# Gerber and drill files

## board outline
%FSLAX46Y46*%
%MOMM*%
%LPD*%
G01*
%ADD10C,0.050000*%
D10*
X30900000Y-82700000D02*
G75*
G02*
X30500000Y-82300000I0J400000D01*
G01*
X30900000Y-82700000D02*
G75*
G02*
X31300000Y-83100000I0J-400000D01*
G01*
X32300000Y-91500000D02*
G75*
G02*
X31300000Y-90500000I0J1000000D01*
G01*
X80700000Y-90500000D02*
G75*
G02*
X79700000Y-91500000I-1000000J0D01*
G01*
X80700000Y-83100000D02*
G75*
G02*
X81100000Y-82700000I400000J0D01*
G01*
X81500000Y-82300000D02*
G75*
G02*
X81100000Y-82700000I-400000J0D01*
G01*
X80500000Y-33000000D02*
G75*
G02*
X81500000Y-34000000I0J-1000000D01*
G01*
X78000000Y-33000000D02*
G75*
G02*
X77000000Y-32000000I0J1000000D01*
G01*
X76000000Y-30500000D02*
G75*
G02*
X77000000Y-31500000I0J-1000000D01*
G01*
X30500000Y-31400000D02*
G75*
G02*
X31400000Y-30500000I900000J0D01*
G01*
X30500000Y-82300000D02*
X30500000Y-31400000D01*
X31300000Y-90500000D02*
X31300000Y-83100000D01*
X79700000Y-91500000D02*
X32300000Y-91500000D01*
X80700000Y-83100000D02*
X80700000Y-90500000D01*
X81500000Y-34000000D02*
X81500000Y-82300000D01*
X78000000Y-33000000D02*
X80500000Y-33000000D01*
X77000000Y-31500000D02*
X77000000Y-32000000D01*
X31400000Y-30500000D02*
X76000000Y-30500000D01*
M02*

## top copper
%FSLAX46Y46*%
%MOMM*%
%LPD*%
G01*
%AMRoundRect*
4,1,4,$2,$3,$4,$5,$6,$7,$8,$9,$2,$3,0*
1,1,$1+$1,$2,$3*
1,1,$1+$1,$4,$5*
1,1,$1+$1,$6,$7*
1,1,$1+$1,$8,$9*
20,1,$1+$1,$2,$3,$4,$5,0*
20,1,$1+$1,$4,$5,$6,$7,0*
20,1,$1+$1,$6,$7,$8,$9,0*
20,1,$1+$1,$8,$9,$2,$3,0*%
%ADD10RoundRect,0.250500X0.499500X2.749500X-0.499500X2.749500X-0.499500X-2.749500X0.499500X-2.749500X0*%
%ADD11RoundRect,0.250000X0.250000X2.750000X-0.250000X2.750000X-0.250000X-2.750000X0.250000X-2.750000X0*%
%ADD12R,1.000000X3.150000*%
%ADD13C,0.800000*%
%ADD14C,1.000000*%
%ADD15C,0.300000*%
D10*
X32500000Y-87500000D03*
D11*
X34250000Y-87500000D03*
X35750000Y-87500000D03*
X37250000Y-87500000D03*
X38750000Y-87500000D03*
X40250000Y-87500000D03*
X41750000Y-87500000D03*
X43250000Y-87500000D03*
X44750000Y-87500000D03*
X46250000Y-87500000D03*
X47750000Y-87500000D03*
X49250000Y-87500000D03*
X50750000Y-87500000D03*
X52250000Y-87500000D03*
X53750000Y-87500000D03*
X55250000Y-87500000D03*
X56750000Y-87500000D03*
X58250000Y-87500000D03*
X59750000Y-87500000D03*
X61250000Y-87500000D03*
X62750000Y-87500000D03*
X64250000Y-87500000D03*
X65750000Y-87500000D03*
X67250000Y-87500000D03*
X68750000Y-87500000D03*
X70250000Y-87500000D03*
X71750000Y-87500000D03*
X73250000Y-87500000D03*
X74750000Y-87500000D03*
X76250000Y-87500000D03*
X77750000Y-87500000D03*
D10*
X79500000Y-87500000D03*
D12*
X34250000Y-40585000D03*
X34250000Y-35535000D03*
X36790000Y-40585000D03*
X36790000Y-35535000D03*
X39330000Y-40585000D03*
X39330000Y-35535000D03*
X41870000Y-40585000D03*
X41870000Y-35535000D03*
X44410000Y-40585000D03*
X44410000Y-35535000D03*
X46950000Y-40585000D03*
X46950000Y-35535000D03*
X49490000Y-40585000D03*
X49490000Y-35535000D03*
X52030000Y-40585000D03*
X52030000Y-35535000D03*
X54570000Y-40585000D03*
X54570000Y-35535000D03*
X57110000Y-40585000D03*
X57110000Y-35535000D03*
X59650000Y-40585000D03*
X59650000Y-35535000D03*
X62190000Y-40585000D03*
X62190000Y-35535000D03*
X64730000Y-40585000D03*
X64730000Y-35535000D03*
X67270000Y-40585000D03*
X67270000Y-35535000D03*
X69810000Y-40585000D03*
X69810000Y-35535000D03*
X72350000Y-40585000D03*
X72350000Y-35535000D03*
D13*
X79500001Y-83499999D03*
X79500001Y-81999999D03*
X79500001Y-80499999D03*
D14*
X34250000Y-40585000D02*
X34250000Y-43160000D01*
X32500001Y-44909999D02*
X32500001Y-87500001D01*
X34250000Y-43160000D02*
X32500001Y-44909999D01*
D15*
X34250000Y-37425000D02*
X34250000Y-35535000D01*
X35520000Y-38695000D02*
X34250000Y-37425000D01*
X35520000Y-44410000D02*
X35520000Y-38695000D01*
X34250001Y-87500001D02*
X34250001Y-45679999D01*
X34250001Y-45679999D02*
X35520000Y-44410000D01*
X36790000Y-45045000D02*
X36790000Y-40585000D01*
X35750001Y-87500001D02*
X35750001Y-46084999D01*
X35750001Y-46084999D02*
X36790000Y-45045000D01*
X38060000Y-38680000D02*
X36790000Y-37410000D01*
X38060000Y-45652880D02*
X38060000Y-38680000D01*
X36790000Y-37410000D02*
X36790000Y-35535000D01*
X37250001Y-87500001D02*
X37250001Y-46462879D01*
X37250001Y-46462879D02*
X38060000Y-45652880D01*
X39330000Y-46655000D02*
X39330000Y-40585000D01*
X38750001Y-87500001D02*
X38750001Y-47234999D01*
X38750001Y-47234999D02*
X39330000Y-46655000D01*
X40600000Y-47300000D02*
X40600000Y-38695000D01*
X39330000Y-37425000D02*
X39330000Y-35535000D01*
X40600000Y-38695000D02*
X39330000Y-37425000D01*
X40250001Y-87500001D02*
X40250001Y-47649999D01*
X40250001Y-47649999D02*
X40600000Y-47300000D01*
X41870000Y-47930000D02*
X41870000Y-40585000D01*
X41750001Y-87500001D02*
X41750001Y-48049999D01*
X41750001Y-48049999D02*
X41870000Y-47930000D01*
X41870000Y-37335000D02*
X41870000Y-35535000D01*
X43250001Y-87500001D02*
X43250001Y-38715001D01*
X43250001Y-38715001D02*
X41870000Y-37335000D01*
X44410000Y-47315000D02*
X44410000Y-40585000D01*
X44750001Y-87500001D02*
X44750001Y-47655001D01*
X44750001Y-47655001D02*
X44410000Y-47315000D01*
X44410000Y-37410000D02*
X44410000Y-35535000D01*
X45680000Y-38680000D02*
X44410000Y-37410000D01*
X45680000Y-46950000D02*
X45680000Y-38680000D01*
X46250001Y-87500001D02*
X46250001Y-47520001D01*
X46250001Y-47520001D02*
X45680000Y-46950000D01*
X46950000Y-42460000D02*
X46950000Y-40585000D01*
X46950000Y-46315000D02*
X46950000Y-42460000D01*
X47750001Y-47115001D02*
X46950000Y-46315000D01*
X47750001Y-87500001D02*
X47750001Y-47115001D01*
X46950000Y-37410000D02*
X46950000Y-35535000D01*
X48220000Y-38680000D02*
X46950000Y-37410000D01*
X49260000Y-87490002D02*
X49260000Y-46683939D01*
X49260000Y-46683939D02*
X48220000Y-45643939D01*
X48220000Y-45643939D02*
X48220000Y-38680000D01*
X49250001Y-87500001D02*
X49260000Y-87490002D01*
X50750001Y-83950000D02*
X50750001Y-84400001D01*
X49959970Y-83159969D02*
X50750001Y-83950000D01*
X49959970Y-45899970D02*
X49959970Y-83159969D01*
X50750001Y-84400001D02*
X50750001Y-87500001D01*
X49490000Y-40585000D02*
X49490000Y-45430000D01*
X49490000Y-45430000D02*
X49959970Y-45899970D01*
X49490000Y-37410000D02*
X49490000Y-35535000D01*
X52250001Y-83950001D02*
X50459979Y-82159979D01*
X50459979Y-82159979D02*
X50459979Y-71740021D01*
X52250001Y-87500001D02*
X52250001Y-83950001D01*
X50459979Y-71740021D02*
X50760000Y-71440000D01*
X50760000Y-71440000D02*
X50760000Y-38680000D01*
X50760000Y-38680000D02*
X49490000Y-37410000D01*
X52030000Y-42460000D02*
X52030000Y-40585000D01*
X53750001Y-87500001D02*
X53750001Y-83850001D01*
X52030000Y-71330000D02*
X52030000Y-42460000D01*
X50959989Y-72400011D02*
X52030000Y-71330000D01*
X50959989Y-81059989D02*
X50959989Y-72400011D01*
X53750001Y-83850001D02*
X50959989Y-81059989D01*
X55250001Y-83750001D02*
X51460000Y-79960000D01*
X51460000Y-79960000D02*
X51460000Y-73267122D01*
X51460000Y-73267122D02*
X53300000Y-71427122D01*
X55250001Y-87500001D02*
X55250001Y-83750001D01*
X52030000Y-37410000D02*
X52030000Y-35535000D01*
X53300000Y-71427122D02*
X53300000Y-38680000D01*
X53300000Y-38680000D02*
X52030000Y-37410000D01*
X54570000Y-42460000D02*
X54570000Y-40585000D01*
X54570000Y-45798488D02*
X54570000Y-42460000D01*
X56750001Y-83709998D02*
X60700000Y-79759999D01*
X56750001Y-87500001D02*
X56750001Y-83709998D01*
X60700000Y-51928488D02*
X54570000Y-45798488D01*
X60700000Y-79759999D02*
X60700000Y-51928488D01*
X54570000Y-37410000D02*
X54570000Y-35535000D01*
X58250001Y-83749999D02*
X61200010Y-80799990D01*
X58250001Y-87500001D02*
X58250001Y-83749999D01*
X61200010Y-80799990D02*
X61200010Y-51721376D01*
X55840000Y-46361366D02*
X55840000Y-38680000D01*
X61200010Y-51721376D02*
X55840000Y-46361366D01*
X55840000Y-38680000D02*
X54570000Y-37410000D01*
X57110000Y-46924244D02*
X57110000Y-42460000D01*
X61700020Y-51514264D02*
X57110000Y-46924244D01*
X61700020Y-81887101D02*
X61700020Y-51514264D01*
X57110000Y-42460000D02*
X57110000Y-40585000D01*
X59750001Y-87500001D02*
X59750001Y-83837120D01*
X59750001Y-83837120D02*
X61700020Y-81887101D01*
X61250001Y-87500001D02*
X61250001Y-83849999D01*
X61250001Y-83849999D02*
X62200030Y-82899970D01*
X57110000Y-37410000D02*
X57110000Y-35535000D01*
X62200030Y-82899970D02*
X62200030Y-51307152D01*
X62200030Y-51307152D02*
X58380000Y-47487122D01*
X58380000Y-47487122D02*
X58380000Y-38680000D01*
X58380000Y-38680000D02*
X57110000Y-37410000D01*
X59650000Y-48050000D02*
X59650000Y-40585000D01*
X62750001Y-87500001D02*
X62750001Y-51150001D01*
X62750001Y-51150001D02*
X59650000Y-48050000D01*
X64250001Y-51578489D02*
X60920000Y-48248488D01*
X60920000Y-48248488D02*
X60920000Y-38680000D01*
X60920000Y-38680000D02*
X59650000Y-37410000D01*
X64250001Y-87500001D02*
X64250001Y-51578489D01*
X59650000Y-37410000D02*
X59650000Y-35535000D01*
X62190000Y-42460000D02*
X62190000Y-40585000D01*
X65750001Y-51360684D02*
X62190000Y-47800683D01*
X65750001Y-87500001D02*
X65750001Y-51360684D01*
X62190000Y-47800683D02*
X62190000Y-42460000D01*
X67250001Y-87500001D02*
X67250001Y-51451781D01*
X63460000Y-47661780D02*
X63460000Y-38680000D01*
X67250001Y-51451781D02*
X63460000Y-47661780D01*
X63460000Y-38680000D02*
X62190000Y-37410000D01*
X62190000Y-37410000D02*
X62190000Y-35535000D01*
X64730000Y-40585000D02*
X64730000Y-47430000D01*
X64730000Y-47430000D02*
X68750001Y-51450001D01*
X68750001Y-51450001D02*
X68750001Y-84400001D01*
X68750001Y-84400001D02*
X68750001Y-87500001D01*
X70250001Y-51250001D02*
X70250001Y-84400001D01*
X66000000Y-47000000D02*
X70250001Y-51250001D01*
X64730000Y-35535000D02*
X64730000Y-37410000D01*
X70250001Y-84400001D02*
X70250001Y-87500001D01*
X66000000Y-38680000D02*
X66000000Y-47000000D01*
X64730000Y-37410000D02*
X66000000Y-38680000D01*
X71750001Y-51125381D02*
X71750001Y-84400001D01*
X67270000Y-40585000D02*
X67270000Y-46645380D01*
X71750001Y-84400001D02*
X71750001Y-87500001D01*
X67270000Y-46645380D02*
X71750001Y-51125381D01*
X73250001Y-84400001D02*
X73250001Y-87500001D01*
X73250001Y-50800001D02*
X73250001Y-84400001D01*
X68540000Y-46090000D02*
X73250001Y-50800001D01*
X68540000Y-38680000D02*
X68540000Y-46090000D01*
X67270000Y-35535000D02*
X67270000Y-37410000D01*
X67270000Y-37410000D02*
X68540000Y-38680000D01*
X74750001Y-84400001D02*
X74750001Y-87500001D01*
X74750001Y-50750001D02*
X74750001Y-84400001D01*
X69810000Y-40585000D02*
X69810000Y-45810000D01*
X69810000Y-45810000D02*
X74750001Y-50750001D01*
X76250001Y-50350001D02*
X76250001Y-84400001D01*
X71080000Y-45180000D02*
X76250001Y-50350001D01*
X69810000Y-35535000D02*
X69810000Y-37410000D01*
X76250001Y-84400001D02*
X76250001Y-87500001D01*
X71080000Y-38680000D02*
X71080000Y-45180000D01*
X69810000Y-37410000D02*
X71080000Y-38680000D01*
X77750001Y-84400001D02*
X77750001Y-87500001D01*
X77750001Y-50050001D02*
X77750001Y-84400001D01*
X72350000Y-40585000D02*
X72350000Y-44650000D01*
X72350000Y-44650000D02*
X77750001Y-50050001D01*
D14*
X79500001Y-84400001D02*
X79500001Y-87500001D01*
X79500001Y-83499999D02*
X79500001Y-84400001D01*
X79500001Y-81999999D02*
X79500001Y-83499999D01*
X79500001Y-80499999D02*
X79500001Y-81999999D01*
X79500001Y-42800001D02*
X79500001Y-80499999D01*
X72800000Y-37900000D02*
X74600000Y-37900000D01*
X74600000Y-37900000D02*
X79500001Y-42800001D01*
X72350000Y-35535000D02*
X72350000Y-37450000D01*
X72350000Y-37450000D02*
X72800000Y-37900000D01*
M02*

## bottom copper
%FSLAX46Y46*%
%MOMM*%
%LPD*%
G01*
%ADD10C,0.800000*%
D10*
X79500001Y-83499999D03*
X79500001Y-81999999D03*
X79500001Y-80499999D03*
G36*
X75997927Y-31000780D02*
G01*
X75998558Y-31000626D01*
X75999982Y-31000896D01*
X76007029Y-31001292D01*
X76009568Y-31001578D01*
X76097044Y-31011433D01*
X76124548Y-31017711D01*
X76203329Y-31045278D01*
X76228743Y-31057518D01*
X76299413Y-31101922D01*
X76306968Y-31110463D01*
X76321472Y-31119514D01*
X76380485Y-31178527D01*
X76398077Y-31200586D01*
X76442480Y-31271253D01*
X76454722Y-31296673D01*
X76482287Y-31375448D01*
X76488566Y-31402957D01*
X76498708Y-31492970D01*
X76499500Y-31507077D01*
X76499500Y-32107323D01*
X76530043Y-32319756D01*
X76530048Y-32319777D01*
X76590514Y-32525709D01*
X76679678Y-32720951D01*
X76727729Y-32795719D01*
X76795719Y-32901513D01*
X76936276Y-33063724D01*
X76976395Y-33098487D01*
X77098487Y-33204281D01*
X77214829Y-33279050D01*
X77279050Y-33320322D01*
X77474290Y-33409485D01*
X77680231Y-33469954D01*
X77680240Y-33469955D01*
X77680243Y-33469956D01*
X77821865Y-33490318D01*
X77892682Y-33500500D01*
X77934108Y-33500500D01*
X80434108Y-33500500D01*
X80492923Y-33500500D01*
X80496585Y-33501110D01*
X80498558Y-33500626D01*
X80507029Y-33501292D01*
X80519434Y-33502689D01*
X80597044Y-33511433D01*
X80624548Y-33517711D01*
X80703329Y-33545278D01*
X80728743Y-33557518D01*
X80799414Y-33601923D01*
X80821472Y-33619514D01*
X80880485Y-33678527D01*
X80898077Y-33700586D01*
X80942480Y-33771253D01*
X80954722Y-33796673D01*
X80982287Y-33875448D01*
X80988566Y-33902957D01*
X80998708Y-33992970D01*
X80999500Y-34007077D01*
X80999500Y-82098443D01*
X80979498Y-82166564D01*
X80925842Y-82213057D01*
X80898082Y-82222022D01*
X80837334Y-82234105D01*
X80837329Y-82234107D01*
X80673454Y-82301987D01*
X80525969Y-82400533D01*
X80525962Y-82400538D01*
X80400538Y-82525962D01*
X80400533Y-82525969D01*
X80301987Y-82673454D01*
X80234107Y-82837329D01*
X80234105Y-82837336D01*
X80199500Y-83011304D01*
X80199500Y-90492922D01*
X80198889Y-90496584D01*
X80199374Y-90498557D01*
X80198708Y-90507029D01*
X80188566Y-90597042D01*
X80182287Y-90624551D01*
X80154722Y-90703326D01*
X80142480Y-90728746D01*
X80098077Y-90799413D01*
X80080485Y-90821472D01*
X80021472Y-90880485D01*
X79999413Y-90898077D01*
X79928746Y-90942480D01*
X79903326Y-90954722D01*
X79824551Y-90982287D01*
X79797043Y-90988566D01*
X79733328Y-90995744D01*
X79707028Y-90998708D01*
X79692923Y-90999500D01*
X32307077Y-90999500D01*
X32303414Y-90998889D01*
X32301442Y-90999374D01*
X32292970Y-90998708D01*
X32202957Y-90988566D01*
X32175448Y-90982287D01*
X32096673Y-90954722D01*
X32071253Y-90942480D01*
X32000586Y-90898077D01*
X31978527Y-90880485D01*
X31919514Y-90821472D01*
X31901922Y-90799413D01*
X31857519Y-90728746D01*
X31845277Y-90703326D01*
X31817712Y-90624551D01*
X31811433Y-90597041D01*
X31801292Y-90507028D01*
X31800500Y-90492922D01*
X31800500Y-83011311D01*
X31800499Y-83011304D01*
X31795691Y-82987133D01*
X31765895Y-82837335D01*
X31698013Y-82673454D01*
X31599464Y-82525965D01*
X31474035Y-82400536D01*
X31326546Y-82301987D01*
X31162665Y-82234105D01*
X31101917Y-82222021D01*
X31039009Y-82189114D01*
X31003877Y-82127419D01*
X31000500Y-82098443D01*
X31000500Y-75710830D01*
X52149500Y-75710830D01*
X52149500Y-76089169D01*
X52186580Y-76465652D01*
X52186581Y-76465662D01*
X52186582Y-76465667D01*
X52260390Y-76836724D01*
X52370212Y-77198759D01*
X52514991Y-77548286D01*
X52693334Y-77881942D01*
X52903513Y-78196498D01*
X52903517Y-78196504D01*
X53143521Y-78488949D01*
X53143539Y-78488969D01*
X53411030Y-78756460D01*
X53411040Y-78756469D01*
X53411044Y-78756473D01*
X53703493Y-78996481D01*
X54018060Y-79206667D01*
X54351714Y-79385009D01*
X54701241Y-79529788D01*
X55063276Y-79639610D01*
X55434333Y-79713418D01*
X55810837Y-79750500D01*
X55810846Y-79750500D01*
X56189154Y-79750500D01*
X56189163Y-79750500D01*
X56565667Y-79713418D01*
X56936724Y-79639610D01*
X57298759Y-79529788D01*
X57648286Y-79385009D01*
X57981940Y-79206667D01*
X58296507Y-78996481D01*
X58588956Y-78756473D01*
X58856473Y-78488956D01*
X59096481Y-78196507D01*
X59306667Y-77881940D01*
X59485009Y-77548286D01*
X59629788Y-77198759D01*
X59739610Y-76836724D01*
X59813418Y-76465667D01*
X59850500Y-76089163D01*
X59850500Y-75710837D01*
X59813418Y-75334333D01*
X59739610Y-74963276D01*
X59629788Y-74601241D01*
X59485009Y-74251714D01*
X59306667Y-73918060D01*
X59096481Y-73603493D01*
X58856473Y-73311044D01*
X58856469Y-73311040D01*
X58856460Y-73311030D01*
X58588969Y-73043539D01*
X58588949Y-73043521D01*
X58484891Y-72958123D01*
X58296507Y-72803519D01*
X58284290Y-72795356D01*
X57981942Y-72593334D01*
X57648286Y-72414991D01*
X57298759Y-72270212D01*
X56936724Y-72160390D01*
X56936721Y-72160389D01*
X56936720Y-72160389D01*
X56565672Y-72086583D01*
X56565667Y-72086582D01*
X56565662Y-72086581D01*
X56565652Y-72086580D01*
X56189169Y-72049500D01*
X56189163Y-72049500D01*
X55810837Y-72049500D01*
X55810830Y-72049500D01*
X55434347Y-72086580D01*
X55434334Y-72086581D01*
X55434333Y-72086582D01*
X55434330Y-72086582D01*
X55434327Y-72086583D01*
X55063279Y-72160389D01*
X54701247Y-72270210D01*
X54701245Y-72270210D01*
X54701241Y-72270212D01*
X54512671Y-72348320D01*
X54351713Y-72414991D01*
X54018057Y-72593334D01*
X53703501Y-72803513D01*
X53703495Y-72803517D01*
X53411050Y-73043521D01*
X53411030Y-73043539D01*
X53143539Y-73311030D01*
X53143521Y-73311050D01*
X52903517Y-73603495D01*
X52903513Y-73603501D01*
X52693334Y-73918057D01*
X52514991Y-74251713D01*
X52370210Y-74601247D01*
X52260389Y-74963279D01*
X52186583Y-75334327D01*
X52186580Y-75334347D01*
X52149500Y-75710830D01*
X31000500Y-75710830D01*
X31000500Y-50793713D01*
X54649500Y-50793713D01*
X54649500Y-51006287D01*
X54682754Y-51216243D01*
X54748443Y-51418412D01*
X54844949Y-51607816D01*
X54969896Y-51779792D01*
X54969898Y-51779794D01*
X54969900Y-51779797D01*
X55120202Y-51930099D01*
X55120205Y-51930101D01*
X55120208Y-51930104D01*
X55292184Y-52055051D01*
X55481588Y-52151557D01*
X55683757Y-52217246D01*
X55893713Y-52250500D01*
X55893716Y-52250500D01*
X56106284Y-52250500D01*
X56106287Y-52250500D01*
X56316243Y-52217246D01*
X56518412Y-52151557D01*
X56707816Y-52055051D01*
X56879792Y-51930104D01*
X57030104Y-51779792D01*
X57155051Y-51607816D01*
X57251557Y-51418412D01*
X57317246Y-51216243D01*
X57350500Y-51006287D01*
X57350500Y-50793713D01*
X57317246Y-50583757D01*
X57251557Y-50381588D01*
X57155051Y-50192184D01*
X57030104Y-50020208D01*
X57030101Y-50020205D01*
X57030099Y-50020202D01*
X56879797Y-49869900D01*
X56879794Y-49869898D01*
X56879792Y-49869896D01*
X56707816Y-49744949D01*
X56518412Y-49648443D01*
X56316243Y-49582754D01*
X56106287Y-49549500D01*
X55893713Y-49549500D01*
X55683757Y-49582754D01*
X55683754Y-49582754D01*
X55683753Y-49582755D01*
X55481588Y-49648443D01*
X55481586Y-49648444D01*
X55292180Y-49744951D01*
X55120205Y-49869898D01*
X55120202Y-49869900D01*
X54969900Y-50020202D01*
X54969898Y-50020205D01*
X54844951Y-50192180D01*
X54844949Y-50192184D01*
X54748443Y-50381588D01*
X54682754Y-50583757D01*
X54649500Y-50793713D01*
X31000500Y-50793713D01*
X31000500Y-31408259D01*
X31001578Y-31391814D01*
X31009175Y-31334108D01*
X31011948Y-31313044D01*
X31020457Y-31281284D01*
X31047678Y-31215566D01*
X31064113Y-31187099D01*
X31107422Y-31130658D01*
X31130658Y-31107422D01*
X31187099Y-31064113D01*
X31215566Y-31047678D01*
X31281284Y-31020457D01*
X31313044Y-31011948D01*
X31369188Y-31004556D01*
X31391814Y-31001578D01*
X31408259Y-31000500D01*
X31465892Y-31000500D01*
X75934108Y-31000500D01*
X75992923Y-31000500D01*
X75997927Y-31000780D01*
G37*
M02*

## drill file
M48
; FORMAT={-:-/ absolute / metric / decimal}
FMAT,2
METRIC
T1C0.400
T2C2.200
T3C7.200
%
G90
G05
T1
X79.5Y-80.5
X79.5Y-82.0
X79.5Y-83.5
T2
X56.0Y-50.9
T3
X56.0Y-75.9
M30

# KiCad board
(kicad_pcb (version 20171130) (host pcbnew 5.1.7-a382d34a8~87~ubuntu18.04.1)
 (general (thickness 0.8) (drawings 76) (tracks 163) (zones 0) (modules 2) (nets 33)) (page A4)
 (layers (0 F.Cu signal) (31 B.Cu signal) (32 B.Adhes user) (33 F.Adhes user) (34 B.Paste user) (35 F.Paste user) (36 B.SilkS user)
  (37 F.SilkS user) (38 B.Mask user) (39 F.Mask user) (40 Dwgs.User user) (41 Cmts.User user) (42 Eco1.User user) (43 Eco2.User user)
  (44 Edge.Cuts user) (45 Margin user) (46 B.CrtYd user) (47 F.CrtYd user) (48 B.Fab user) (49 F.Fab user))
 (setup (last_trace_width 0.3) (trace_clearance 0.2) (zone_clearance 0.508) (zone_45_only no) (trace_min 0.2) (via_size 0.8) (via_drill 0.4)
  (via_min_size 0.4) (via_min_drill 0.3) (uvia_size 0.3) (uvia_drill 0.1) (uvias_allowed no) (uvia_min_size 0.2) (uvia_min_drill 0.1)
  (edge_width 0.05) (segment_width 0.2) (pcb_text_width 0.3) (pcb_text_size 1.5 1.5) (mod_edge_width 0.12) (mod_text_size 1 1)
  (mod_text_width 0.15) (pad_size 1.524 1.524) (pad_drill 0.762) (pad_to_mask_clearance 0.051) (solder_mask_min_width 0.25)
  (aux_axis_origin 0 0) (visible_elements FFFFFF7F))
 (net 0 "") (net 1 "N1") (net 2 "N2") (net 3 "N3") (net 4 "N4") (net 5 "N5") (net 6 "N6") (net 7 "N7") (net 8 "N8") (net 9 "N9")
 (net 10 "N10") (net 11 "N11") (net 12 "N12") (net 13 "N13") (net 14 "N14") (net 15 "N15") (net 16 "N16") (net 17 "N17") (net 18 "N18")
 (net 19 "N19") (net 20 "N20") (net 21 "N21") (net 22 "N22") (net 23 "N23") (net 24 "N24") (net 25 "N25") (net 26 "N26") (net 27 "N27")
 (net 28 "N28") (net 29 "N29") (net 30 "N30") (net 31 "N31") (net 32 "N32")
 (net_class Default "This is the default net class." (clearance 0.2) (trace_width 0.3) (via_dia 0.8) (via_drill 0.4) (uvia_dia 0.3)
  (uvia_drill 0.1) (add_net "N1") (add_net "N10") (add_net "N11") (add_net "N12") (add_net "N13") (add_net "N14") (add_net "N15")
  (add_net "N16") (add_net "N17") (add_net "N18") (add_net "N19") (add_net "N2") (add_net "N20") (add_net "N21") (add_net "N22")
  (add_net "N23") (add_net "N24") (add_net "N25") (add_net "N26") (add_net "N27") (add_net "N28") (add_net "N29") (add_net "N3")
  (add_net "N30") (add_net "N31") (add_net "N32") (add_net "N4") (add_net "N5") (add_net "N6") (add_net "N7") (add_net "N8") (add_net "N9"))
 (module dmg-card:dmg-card (layer F.Cu) (at 56 61)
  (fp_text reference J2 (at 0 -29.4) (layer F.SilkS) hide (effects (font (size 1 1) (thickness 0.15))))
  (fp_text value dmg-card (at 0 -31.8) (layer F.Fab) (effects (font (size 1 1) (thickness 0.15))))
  (pad 1 smd roundrect (at -23.5 26.5 180) (size 1.5 6) (layers F.Cu) (roundrect_rratio 0.167) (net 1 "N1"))
  (pad 2 smd roundrect (at -21.75 26.5 180) (size 1 6) (layers F.Cu) (roundrect_rratio 0.25) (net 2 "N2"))
  (pad 3 smd roundrect (at -20.25 26.5 180) (size 1 6) (layers F.Cu) (roundrect_rratio 0.25) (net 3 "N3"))
  (pad 4 smd roundrect (at -18.75 26.5 180) (size 1 6) (layers F.Cu) (roundrect_rratio 0.25) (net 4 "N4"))
  (pad 5 smd roundrect (at -17.25 26.5 180) (size 1 6) (layers F.Cu) (roundrect_rratio 0.25) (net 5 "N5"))
  (pad 6 smd roundrect (at -15.75 26.5 180) (size 1 6) (layers F.Cu) (roundrect_rratio 0.25) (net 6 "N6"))
  (pad 7 smd roundrect (at -14.25 26.5 180) (size 1 6) (layers F.Cu) (roundrect_rratio 0.25) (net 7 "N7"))
  (pad 8 smd roundrect (at -12.75 26.5 180) (size 1 6) (layers F.Cu) (roundrect_rratio 0.25) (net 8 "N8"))
  (pad 9 smd roundrect (at -11.25 26.5 180) (size 1 6) (layers F.Cu) (roundrect_rratio 0.25) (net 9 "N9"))
  (pad 10 smd roundrect (at -9.75 26.5 180) (size 1 6) (layers F.Cu) (roundrect_rratio 0.25) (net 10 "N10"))
  (pad 11 smd roundrect (at -8.25 26.5 180) (size 1 6) (layers F.Cu) (roundrect_rratio 0.25) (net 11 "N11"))
  (pad 12 smd roundrect (at -6.75 26.5 180) (size 1 6) (layers F.Cu) (roundrect_rratio 0.25) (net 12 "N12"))
  (pad 13 smd roundrect (at -5.25 26.5 180) (size 1 6) (layers F.Cu) (roundrect_rratio 0.25) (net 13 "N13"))
  (pad 14 smd roundrect (at -3.75 26.5 180) (size 1 6) (layers F.Cu) (roundrect_rratio 0.25) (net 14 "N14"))
  (pad 15 smd roundrect (at -2.25 26.5 180) (size 1 6) (layers F.Cu) (roundrect_rratio 0.25) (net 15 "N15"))
  (pad 16 smd roundrect (at -0.75 26.5 180) (size 1 6) (layers F.Cu) (roundrect_rratio 0.25) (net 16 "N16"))
  (pad 17 smd roundrect (at 0.75 26.5 180) (size 1 6) (layers F.Cu) (roundrect_rratio 0.25) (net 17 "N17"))
  (pad 18 smd roundrect (at 2.25 26.5 180) (size 1 6) (layers F.Cu) (roundrect_rratio 0.25) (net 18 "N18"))
  (pad 19 smd roundrect (at 3.75 26.5 180) (size 1 6) (layers F.Cu) (roundrect_rratio 0.25) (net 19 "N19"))
  (pad 20 smd roundrect (at 5.25 26.5 180) (size 1 6) (layers F.Cu) (roundrect_rratio 0.25) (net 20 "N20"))
  (pad 21 smd roundrect (at 6.75 26.5 180) (size 1 6) (layers F.Cu) (roundrect_rratio 0.25) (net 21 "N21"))
  (pad 22 smd roundrect (at 8.25 26.5 180) (size 1 6) (layers F.Cu) (roundrect_rratio 0.25) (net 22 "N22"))
  (pad 23 smd roundrect (at 9.75 26.5 180) (size 1 6) (layers F.Cu) (roundrect_rratio 0.25) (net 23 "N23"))
  (pad 24 smd roundrect (at 11.25 26.5 180) (size 1 6) (layers F.Cu) (roundrect_rratio 0.25) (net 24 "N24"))
  (pad 25 smd roundrect (at 12.75 26.5 180) (size 1 6) (layers F.Cu) (roundrect_rratio 0.25) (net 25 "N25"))
  (pad 26 smd roundrect (at 14.25 26.5 180) (size 1 6) (layers F.Cu) (roundrect_rratio 0.25) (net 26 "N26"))
  (pad 27 smd roundrect (at 15.75 26.5 180) (size 1 6) (layers F.Cu) (roundrect_rratio 0.25) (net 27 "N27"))
  (pad 28 smd roundrect (at 17.25 26.5 180) (size 1 6) (layers F.Cu) (roundrect_rratio 0.25) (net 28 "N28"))
  (pad 29 smd roundrect (at 18.75 26.5 180) (size 1 6) (layers F.Cu) (roundrect_rratio 0.25) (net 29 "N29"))
  (pad 30 smd roundrect (at 20.25 26.5 180) (size 1 6) (layers F.Cu) (roundrect_rratio 0.25) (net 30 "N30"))
  (pad 31 smd roundrect (at 21.75 26.5 180) (size 1 6) (layers F.Cu) (roundrect_rratio 0.25) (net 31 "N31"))
  (pad 32 smd roundrect (at 23.5 26.5 180) (size 1.5 6) (layers F.Cu) (roundrect_rratio 0.167) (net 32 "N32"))
  (pad MASK0 smd roundrect (at 0 27.5 180) (size 49.4 6) (layers F.Mask) (roundrect_rratio 0.167))
  (pad 33 smd rect (at 0 25.5 180) (size 49.4 3) (layers F.Mask))
  (pad "" np_thru_hole circle (at 0 14.9) (size 7.2 7.2) (drill 7.2) (layers *.Cu *.Mask))
  (pad "" np_thru_hole circle (at 0 -10.1) (size 2.2 2.2) (drill 2.2) (layers *.Cu *.Mask)))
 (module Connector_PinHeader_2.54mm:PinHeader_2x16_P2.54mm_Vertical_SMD (layer F.Cu) (at 53.3 38.06 90)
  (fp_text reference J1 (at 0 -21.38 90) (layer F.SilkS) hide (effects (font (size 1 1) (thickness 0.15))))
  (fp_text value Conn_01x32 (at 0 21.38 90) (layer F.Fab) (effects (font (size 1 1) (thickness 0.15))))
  (pad 1 smd rect (at -2.525 -19.05 90) (size 3.15 1) (layers F.Cu F.Paste F.Mask) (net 1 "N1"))
  (pad 2 smd rect (at 2.525 -19.05 90) (size 3.15 1) (layers F.Cu F.Paste F.Mask) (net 2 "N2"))
  (pad 3 smd rect (at -2.525 -16.51 90) (size 3.15 1) (layers F.Cu F.Paste F.Mask) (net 3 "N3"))
  (pad 4 smd rect (at 2.525 -16.51 90) (size 3.15 1) (layers F.Cu F.Paste F.Mask) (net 4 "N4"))
  (pad 5 smd rect (at -2.525 -13.97 90) (size 3.15 1) (layers F.Cu F.Paste F.Mask) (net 5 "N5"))
  (pad 6 smd rect (at 2.525 -13.97 90) (size 3.15 1) (layers F.Cu F.Paste F.Mask) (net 6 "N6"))
  (pad 7 smd rect (at -2.525 -11.43 90) (size 3.15 1) (layers F.Cu F.Paste F.Mask) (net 7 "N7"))
  (pad 8 smd rect (at 2.525 -11.43 90) (size 3.15 1) (layers F.Cu F.Paste F.Mask) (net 8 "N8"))
  (pad 9 smd rect (at -2.525 -8.89 90) (size 3.15 1) (layers F.Cu F.Paste F.Mask) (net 9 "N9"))
  (pad 10 smd rect (at 2.525 -8.89 90) (size 3.15 1) (layers F.Cu F.Paste F.Mask) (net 10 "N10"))
  (pad 11 smd rect (at -2.525 -6.35 90) (size 3.15 1) (layers F.Cu F.Paste F.Mask) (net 11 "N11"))
  (pad 12 smd rect (at 2.525 -6.35 90) (size 3.15 1) (layers F.Cu F.Paste F.Mask) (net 12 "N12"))
  (pad 13 smd rect (at -2.525 -3.81 90) (size 3.15 1) (layers F.Cu F.Paste F.Mask) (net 13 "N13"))
  (pad 14 smd rect (at 2.525 -3.81 90) (size 3.15 1) (layers F.Cu F.Paste F.Mask) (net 14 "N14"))
  (pad 15 smd rect (at -2.525 -1.27 90) (size 3.15 1) (layers F.Cu F.Paste F.Mask) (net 15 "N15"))
  (pad 16 smd rect (at 2.525 -1.27 90) (size 3.15 1) (layers F.Cu F.Paste F.Mask) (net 16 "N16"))
  (pad 17 smd rect (at -2.525 1.27 90) (size 3.15 1) (layers F.Cu F.Paste F.Mask) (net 17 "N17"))
  (pad 18 smd rect (at 2.525 1.27 90) (size 3.15 1) (layers F.Cu F.Paste F.Mask) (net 18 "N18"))
  (pad 19 smd rect (at -2.525 3.81 90) (size 3.15 1) (layers F.Cu F.Paste F.Mask) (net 19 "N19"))
  (pad 20 smd rect (at 2.525 3.81 90) (size 3.15 1) (layers F.Cu F.Paste F.Mask) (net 20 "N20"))
  (pad 21 smd rect (at -2.525 6.35 90) (size 3.15 1) (layers F.Cu F.Paste F.Mask) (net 21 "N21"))
  (pad 22 smd rect (at 2.525 6.35 90) (size 3.15 1) (layers F.Cu F.Paste F.Mask) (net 22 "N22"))
  (pad 23 smd rect (at -2.525 8.89 90) (size 3.15 1) (layers F.Cu F.Paste F.Mask) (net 23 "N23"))
  (pad 24 smd rect (at 2.525 8.89 90) (size 3.15 1) (layers F.Cu F.Paste F.Mask) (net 24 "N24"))
  (pad 25 smd rect (at -2.525 11.43 90) (size 3.15 1) (layers F.Cu F.Paste F.Mask) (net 25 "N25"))
  (pad 26 smd rect (at 2.525 11.43 90) (size 3.15 1) (layers F.Cu F.Paste F.Mask) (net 26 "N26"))
  (pad 27 smd rect (at -2.525 13.97 90) (size 3.15 1) (layers F.Cu F.Paste F.Mask) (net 27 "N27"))
  (pad 28 smd rect (at 2.525 13.97 90) (size 3.15 1) (layers F.Cu F.Paste F.Mask) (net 28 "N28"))
  (pad 29 smd rect (at -2.525 16.51 90) (size 3.15 1) (layers F.Cu F.Paste F.Mask) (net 29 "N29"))
  (pad 30 smd rect (at 2.525 16.51 90) (size 3.15 1) (layers F.Cu F.Paste F.Mask) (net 30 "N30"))
  (pad 31 smd rect (at -2.525 19.05 90) (size 3.15 1) (layers F.Cu F.Paste F.Mask) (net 31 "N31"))
  (pad 32 smd rect (at 2.525 19.05 90) (size 3.15 1) (layers F.Cu F.Paste F.Mask) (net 32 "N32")))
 (gr_arc (start 30.9 82.3) (end 30.5 82.3) (angle -90) (layer Edge.Cuts) (width 0.05))
 (gr_arc (start 30.9 83.1) (end 31.3 83.1) (angle -90) (layer Edge.Cuts) (width 0.05))
 (gr_arc (start 32.3 90.5) (end 31.3 90.5) (angle -90) (layer Edge.Cuts) (width 0.05))
 (gr_arc (start 79.7 90.5) (end 79.7 91.5) (angle -90) (layer Edge.Cuts) (width 0.05))
 (gr_arc (start 81.1 83.1) (end 81.1 82.7) (angle -90) (layer Edge.Cuts) (width 0.05))
 (gr_arc (start 81.1 82.3) (end 81.1 82.7) (angle -90) (layer Edge.Cuts) (width 0.05))
 (gr_arc (start 80.5 34) (end 81.5 34) (angle -90) (layer Edge.Cuts) (width 0.05))
 (gr_arc (start 78 32) (end 77 32) (angle -90) (layer Edge.Cuts) (width 0.05))
 (gr_arc (start 76 31.5) (end 77 31.5) (angle -90) (layer Edge.Cuts) (width 0.05))
 (gr_arc (start 31.4 31.4) (end 31.4 30.5) (angle -90) (layer Edge.Cuts) (width 0.05))
 (gr_line (start 30.5 82.3) (end 30.5 31.4) (layer Edge.Cuts) (width 0.05))
 (gr_line (start 31.3 90.5) (end 31.3 83.1) (layer Edge.Cuts) (width 0.05))
 (gr_line (start 79.7 91.5) (end 32.3 91.5) (layer Edge.Cuts) (width 0.05))
 (gr_line (start 80.7 83.1) (end 80.7 90.5) (layer Edge.Cuts) (width 0.05))
 (gr_line (start 81.5 34) (end 81.5 82.3) (layer Edge.Cuts) (width 0.05))
 (gr_line (start 78 33) (end 80.5 33) (layer Edge.Cuts) (width 0.05))
 (gr_line (start 77 31.5) (end 77 32) (layer Edge.Cuts) (width 0.05))
 (gr_line (start 31.4 30.5) (end 76 30.5) (layer Edge.Cuts) (width 0.05))
 (segment (start 34.25 40.585) (end 34.25 43.16) (width 1) (layer F.Cu) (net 1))
 (segment (start 32.500001 44.909999) (end 32.500001 87.500001) (width 1) (layer F.Cu) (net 1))
 (segment (start 34.25 43.16) (end 32.500001 44.909999) (width 1) (layer F.Cu) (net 1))
 (segment (start 34.25 37.425) (end 34.25 35.535) (width 0.3) (layer F.Cu) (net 2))
 (segment (start 35.52 38.695) (end 34.25 37.425) (width 0.3) (layer F.Cu) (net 2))
 (segment (start 35.52 44.41) (end 35.52 38.695) (width 0.3) (layer F.Cu) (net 2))
 (segment (start 34.250001 87.500001) (end 34.250001 45.679999) (width 0.3) (layer F.Cu) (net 2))
 (segment (start 34.250001 45.679999) (end 35.52 44.41) (width 0.3) (layer F.Cu) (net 2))
 (segment (start 36.79 45.045) (end 36.79 40.585) (width 0.3) (layer F.Cu) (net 3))
 (segment (start 35.750001 87.500001) (end 35.750001 46.084999) (width 0.3) (layer F.Cu) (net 3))
 (segment (start 35.750001 46.084999) (end 36.79 45.045) (width 0.3) (layer F.Cu) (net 3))
 (segment (start 38.06 38.68) (end 36.79 37.41) (width 0.3) (layer F.Cu) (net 4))
 (segment (start 38.06 45.65288) (end 38.06 38.68) (width 0.3) (layer F.Cu) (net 4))
 (segment (start 36.79 37.41) (end 36.79 35.535) (width 0.3) (layer F.Cu) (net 4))
 (segment (start 37.250001 87.500001) (end 37.250001 46.462879) (width 0.3) (layer F.Cu) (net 4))
 (segment (start 37.250001 46.462879) (end 38.06 45.65288) (width 0.3) (layer F.Cu) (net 4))
 (segment (start 39.33 46.655) (end 39.33 40.585) (width 0.3) (layer F.Cu) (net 5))
 (segment (start 38.750001 87.500001) (end 38.750001 47.234999) (width 0.3) (layer F.Cu) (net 5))
 (segment (start 38.750001 47.234999) (end 39.33 46.655) (width 0.3) (layer F.Cu) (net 5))
 (segment (start 40.6 47.3) (end 40.6 38.695) (width 0.3) (layer F.Cu) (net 6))
 (segment (start 39.33 37.425) (end 39.33 35.535) (width 0.3) (layer F.Cu) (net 6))
 (segment (start 40.6 38.695) (end 39.33 37.425) (width 0.3) (layer F.Cu) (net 6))
 (segment (start 40.250001 87.500001) (end 40.250001 47.649999) (width 0.3) (layer F.Cu) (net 6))
 (segment (start 40.250001 47.649999) (end 40.6 47.3) (width 0.3) (layer F.Cu) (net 6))
 (segment (start 41.87 47.93) (end 41.87 40.585) (width 0.3) (layer F.Cu) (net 7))
 (segment (start 41.750001 87.500001) (end 41.750001 48.049999) (width 0.3) (layer F.Cu) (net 7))
 (segment (start 41.750001 48.049999) (end 41.87 47.93) (width 0.3) (layer F.Cu) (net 7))
 (segment (start 41.87 37.335) (end 41.87 35.535) (width 0.3) (layer F.Cu) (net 8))
 (segment (start 43.250001 87.500001) (end 43.250001 38.715001) (width 0.3) (layer F.Cu) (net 8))
 (segment (start 43.250001 38.715001) (end 41.87 37.335) (width 0.3) (layer F.Cu) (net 8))
 (segment (start 44.41 47.315) (end 44.41 40.585) (width 0.3) (layer F.Cu) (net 9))
 (segment (start 44.750001 87.500001) (end 44.750001 47.655001) (width 0.3) (layer F.Cu) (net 9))
 (segment (start 44.750001 47.655001) (end 44.41 47.315) (width 0.3) (layer F.Cu) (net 9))
 (segment (start 44.41 37.41) (end 44.41 35.535) (width 0.3) (layer F.Cu) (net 10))
 (segment (start 45.68 38.68) (end 44.41 37.41) (width 0.3) (layer F.Cu) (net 10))
 (segment (start 45.68 46.95) (end 45.68 38.68) (width 0.3) (layer F.Cu) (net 10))
 (segment (start 46.250001 87.500001) (end 46.250001 47.520001) (width 0.3) (layer F.Cu) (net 10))
 (segment (start 46.250001 47.520001) (end 45.68 46.95) (width 0.3) (layer F.Cu) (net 10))
 (segment (start 46.95 42.46) (end 46.95 40.585) (width 0.3) (layer F.Cu) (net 11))
 (segment (start 46.95 46.315) (end 46.95 42.46) (width 0.3) (layer F.Cu) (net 11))
 (segment (start 47.750001 47.115001) (end 46.95 46.315) (width 0.3) (layer F.Cu) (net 11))
 (segment (start 47.750001 87.500001) (end 47.750001 47.115001) (width 0.3) (layer F.Cu) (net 11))
 (segment (start 46.95 37.41) (end 46.95 35.535) (width 0.3) (layer F.Cu) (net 12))
 (segment (start 48.22 38.68) (end 46.95 37.41) (width 0.3) (layer F.Cu) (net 12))
 (segment (start 49.26 87.490002) (end 49.26 46.683939) (width 0.3) (layer F.Cu) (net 12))
 (segment (start 49.26 46.683939) (end 48.22 45.643939) (width 0.3) (layer F.Cu) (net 12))
 (segment (start 48.22 45.643939) (end 48.22 38.68) (width 0.3) (layer F.Cu) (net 12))
 (segment (start 49.250001 87.500001) (end 49.26 87.490002) (width 0.3) (layer F.Cu) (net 12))
 (segment (start 50.750001 83.95) (end 50.750001 84.400001) (width 0.3) (layer F.Cu) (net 13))
 (segment (start 49.95997 83.159969) (end 50.750001 83.95) (width 0.3) (layer F.Cu) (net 13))
 (segment (start 49.95997 45.89997) (end 49.95997 83.159969) (width 0.3) (layer F.Cu) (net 13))
 (segment (start 50.750001 84.400001) (end 50.750001 87.500001) (width 0.3) (layer F.Cu) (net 13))
 (segment (start 49.49 40.585) (end 49.49 45.43) (width 0.3) (layer F.Cu) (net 13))
 (segment (start 49.49 45.43) (end 49.95997 45.89997) (width 0.3) (layer F.Cu) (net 13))
 (segment (start 49.49 37.41) (end 49.49 35.535) (width 0.3) (layer F.Cu) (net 14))
 (segment (start 52.250001 83.950001) (end 50.459979 82.159979) (width 0.3) (layer F.Cu) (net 14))
 (segment (start 50.459979 82.159979) (end 50.459979 71.740021) (width 0.3) (layer F.Cu) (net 14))
 (segment (start 52.250001 87.500001) (end 52.250001 83.950001) (width 0.3) (layer F.Cu) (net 14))
 (segment (start 50.459979 71.740021) (end 50.76 71.44) (width 0.3) (layer F.Cu) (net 14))
 (segment (start 50.76 71.44) (end 50.76 38.68) (width 0.3) (layer F.Cu) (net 14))
 (segment (start 50.76 38.68) (end 49.49 37.41) (width 0.3) (layer F.Cu) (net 14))
 (segment (start 52.03 42.46) (end 52.03 40.585) (width 0.3) (layer F.Cu) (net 15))
 (segment (start 53.750001 87.500001) (end 53.750001 83.850001) (width 0.3) (layer F.Cu) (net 15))
 (segment (start 52.03 71.33) (end 52.03 42.46) (width 0.3) (layer F.Cu) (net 15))
 (segment (start 50.959989 72.400011) (end 52.03 71.33) (width 0.3) (layer F.Cu) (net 15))
 (segment (start 50.959989 81.059989) (end 50.959989 72.400011) (width 0.3) (layer F.Cu) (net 15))
 (segment (start 53.750001 83.850001) (end 50.959989 81.059989) (width 0.3) (layer F.Cu) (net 15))
 (segment (start 55.250001 83.750001) (end 51.46 79.96) (width 0.3) (layer F.Cu) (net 16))
 (segment (start 51.46 79.96) (end 51.46 73.267122) (width 0.3) (layer F.Cu) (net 16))
 (segment (start 51.46 73.267122) (end 53.3 71.427122) (width 0.3) (layer F.Cu) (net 16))
 (segment (start 55.250001 87.500001) (end 55.250001 83.750001) (width 0.3) (layer F.Cu) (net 16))
 (segment (start 52.03 37.41) (end 52.03 35.535) (width 0.3) (layer F.Cu) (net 16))
 (segment (start 53.3 71.427122) (end 53.3 38.68) (width 0.3) (layer F.Cu) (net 16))
 (segment (start 53.3 38.68) (end 52.03 37.41) (width 0.3) (layer F.Cu) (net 16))
 (segment (start 54.57 42.46) (end 54.57 40.585) (width 0.3) (layer F.Cu) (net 17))
 (segment (start 54.57 45.798488) (end 54.57 42.46) (width 0.3) (layer F.Cu) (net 17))
 (segment (start 56.750001 83.709998) (end 60.7 79.759999) (width 0.3) (layer F.Cu) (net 17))
 (segment (start 56.750001 87.500001) (end 56.750001 83.709998) (width 0.3) (layer F.Cu) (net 17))
 (segment (start 60.7 51.928488) (end 54.57 45.798488) (width 0.3) (layer F.Cu) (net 17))
 (segment (start 60.7 79.759999) (end 60.7 51.928488) (width 0.3) (layer F.Cu) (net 17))
 (segment (start 54.57 37.41) (end 54.57 35.535) (width 0.3) (layer F.Cu) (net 18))
 (segment (start 58.250001 83.749999) (end 61.20001 80.79999) (width 0.3) (layer F.Cu) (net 18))
 (segment (start 58.250001 87.500001) (end 58.250001 83.749999) (width 0.3) (layer F.Cu) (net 18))
 (segment (start 61.20001 80.79999) (end 61.20001 51.721376) (width 0.3) (layer F.Cu) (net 18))
 (segment (start 55.84 46.361366) (end 55.84 38.68) (width 0.3) (layer F.Cu) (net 18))
 (segment (start 61.20001 51.721376) (end 55.84 46.361366) (width 0.3) (layer F.Cu) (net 18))
 (segment (start 55.84 38.68) (end 54.57 37.41) (width 0.3) (layer F.Cu) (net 18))
 (segment (start 57.11 46.924244) (end 57.11 42.46) (width 0.3) (layer F.Cu) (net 19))
 (segment (start 61.70002 51.514264) (end 57.11 46.924244) (width 0.3) (layer F.Cu) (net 19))
 (segment (start 61.70002 81.887101) (end 61.70002 51.514264) (width 0.3) (layer F.Cu) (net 19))
 (segment (start 57.11 42.46) (end 57.11 40.585) (width 0.3) (layer F.Cu) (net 19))
 (segment (start 59.750001 87.500001) (end 59.750001 83.83712) (width 0.3) (layer F.Cu) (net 19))
 (segment (start 59.750001 83.83712) (end 61.70002 81.887101) (width 0.3) (layer F.Cu) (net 19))
 (segment (start 61.250001 87.500001) (end 61.250001 83.849999) (width 0.3) (layer F.Cu) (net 20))
 (segment (start 61.250001 83.849999) (end 62.20003 82.89997) (width 0.3) (layer F.Cu) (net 20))
 (segment (start 57.11 37.41) (end 57.11 35.535) (width 0.3) (layer F.Cu) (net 20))
 (segment (start 62.20003 82.89997) (end 62.20003 51.307152) (width 0.3) (layer F.Cu) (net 20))
 (segment (start 62.20003 51.307152) (end 58.38 47.487122) (width 0.3) (layer F.Cu) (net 20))
 (segment (start 58.38 47.487122) (end 58.38 38.68) (width 0.3) (layer F.Cu) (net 20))
 (segment (start 58.38 38.68) (end 57.11 37.41) (width 0.3) (layer F.Cu) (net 20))
 (segment (start 59.65 48.05) (end 59.65 40.585) (width 0.3) (layer F.Cu) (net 21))
 (segment (start 62.750001 87.500001) (end 62.750001 51.150001) (width 0.3) (layer F.Cu) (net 21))
 (segment (start 62.750001 51.150001) (end 59.65 48.05) (width 0.3) (layer F.Cu) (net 21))
 (segment (start 64.250001 51.578489) (end 60.92 48.248488) (width 0.3) (layer F.Cu) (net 22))
 (segment (start 60.92 48.248488) (end 60.92 38.68) (width 0.3) (layer F.Cu) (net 22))
 (segment (start 60.92 38.68) (end 59.65 37.41) (width 0.3) (layer F.Cu) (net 22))
 (segment (start 64.250001 87.500001) (end 64.250001 51.578489) (width 0.3) (layer F.Cu) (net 22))
 (segment (start 59.65 37.41) (end 59.65 35.535) (width 0.3) (layer F.Cu) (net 22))
 (segment (start 62.19 42.46) (end 62.19 40.585) (width 0.3) (layer F.Cu) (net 23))
 (segment (start 65.750001 51.360684) (end 62.19 47.800683) (width 0.3) (layer F.Cu) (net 23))
 (segment (start 65.750001 87.500001) (end 65.750001 51.360684) (width 0.3) (layer F.Cu) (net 23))
 (segment (start 62.19 47.800683) (end 62.19 42.46) (width 0.3) (layer F.Cu) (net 23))
 (segment (start 67.250001 87.500001) (end 67.250001 51.451781) (width 0.3) (layer F.Cu) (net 24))
 (segment (start 63.46 47.66178) (end 63.46 38.68) (width 0.3) (layer F.Cu) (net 24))
 (segment (start 67.250001 51.451781) (end 63.46 47.66178) (width 0.3) (layer F.Cu) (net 24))
 (segment (start 63.46 38.68) (end 62.19 37.41) (width 0.3) (layer F.Cu) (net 24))
 (segment (start 62.19 37.41) (end 62.19 35.535) (width 0.3) (layer F.Cu) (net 24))
 (segment (start 64.73 40.585) (end 64.73 47.43) (width 0.3) (layer F.Cu) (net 25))
 (segment (start 64.73 47.43) (end 68.750001 51.450001) (width 0.3) (layer F.Cu) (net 25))
 (segment (start 68.750001 51.450001) (end 68.750001 84.400001) (width 0.3) (layer F.Cu) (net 25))
 (segment (start 68.750001 84.400001) (end 68.750001 87.500001) (width 0.3) (layer F.Cu) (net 25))
 (segment (start 70.250001 51.250001) (end 70.250001 84.400001) (width 0.3) (layer F.Cu) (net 26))
 (segment (start 66 47) (end 70.250001 51.250001) (width 0.3) (layer F.Cu) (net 26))
 (segment (start 64.73 35.535) (end 64.73 37.41) (width 0.3) (layer F.Cu) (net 26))
 (segment (start 70.250001 84.400001) (end 70.250001 87.500001) (width 0.3) (layer F.Cu) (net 26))
 (segment (start 66 38.68) (end 66 47) (width 0.3) (layer F.Cu) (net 26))
 (segment (start 64.73 37.41) (end 66 38.68) (width 0.3) (layer F.Cu) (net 26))
 (segment (start 71.750001 51.125381) (end 71.750001 84.400001) (width 0.3) (layer F.Cu) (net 27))
 (segment (start 67.27 40.585) (end 67.27 46.64538) (width 0.3) (layer F.Cu) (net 27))
 (segment (start 71.750001 84.400001) (end 71.750001 87.500001) (width 0.3) (layer F.Cu) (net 27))
 (segment (start 67.27 46.64538) (end 71.750001 51.125381) (width 0.3) (layer F.Cu) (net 27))
 (segment (start 73.250001 84.400001) (end 73.250001 87.500001) (width 0.3) (layer F.Cu) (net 28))
 (segment (start 73.250001 50.800001) (end 73.250001 84.400001) (width 0.3) (layer F.Cu) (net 28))
 (segment (start 68.54 46.09) (end 73.250001 50.800001) (width 0.3) (layer F.Cu) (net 28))
 (segment (start 68.54 38.68) (end 68.54 46.09) (width 0.3) (layer F.Cu) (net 28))
 (segment (start 67.27 35.535) (end 67.27 37.41) (width 0.3) (layer F.Cu) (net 28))
 (segment (start 67.27 37.41) (end 68.54 38.68) (width 0.3) (layer F.Cu) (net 28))
 (segment (start 74.750001 84.400001) (end 74.750001 87.500001) (width 0.3) (layer F.Cu) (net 29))
 (segment (start 74.750001 50.750001) (end 74.750001 84.400001) (width 0.3) (layer F.Cu) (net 29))
 (segment (start 69.81 40.585) (end 69.81 45.81) (width 0.3) (layer F.Cu) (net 29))
 (segment (start 69.81 45.81) (end 74.750001 50.750001) (width 0.3) (layer F.Cu) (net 29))
 (segment (start 76.250001 50.350001) (end 76.250001 84.400001) (width 0.3) (layer F.Cu) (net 30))
 (segment (start 71.08 45.18) (end 76.250001 50.350001) (width 0.3) (layer F.Cu) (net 30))
 (segment (start 69.81 35.535) (end 69.81 37.41) (width 0.3) (layer F.Cu) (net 30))
 (segment (start 76.250001 84.400001) (end 76.250001 87.500001) (width 0.3) (layer F.Cu) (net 30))
 (segment (start 71.08 38.68) (end 71.08 45.18) (width 0.3) (layer F.Cu) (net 30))
 (segment (start 69.81 37.41) (end 71.08 38.68) (width 0.3) (layer F.Cu) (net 30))
 (segment (start 77.750001 84.400001) (end 77.750001 87.500001) (width 0.3) (layer F.Cu) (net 31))
 (segment (start 77.750001 50.050001) (end 77.750001 84.400001) (width 0.3) (layer F.Cu) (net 31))
 (segment (start 72.35 40.585) (end 72.35 44.65) (width 0.3) (layer F.Cu) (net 31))
 (segment (start 72.35 44.65) (end 77.750001 50.050001) (width 0.3) (layer F.Cu) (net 31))
 (segment (start 79.500001 84.400001) (end 79.500001 87.500001) (width 1) (layer F.Cu) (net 32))
 (segment (start 79.500001 83.499999) (end 79.500001 84.400001) (width 1) (layer F.Cu) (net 32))
 (via (at 79.500001 83.499999) (size 0.8) (drill 0.4) (layers F.Cu B.Cu) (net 32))
 (segment (start 79.500001 81.999999) (end 79.500001 83.499999) (width 1) (layer F.Cu) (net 32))
 (via (at 79.500001 81.999999) (size 0.8) (drill 0.4) (layers F.Cu B.Cu) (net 32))
 (segment (start 79.500001 80.499999) (end 79.500001 81.999999) (width 1) (layer F.Cu) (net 32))
 (via (at 79.500001 80.499999) (size 0.8) (drill 0.4) (layers F.Cu B.Cu) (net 32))
 (segment (start 79.500001 42.800001) (end 79.500001 80.499999) (width 1) (layer F.Cu) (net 32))
 (segment (start 72.8 37.9) (end 74.6 37.9) (width 1) (layer F.Cu) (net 32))
 (segment (start 74.6 37.9) (end 79.500001 42.800001) (width 1) (layer F.Cu) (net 32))
 (segment (start 72.35 35.535) (end 72.35 37.45) (width 1) (layer F.Cu) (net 32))
 (segment (start 72.35 37.45) (end 72.8 37.9) (width 1) (layer F.Cu) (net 32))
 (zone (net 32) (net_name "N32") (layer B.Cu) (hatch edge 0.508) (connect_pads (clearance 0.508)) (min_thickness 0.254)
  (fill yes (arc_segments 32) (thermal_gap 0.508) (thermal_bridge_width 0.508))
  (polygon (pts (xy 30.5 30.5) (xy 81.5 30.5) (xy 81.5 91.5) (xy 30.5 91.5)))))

